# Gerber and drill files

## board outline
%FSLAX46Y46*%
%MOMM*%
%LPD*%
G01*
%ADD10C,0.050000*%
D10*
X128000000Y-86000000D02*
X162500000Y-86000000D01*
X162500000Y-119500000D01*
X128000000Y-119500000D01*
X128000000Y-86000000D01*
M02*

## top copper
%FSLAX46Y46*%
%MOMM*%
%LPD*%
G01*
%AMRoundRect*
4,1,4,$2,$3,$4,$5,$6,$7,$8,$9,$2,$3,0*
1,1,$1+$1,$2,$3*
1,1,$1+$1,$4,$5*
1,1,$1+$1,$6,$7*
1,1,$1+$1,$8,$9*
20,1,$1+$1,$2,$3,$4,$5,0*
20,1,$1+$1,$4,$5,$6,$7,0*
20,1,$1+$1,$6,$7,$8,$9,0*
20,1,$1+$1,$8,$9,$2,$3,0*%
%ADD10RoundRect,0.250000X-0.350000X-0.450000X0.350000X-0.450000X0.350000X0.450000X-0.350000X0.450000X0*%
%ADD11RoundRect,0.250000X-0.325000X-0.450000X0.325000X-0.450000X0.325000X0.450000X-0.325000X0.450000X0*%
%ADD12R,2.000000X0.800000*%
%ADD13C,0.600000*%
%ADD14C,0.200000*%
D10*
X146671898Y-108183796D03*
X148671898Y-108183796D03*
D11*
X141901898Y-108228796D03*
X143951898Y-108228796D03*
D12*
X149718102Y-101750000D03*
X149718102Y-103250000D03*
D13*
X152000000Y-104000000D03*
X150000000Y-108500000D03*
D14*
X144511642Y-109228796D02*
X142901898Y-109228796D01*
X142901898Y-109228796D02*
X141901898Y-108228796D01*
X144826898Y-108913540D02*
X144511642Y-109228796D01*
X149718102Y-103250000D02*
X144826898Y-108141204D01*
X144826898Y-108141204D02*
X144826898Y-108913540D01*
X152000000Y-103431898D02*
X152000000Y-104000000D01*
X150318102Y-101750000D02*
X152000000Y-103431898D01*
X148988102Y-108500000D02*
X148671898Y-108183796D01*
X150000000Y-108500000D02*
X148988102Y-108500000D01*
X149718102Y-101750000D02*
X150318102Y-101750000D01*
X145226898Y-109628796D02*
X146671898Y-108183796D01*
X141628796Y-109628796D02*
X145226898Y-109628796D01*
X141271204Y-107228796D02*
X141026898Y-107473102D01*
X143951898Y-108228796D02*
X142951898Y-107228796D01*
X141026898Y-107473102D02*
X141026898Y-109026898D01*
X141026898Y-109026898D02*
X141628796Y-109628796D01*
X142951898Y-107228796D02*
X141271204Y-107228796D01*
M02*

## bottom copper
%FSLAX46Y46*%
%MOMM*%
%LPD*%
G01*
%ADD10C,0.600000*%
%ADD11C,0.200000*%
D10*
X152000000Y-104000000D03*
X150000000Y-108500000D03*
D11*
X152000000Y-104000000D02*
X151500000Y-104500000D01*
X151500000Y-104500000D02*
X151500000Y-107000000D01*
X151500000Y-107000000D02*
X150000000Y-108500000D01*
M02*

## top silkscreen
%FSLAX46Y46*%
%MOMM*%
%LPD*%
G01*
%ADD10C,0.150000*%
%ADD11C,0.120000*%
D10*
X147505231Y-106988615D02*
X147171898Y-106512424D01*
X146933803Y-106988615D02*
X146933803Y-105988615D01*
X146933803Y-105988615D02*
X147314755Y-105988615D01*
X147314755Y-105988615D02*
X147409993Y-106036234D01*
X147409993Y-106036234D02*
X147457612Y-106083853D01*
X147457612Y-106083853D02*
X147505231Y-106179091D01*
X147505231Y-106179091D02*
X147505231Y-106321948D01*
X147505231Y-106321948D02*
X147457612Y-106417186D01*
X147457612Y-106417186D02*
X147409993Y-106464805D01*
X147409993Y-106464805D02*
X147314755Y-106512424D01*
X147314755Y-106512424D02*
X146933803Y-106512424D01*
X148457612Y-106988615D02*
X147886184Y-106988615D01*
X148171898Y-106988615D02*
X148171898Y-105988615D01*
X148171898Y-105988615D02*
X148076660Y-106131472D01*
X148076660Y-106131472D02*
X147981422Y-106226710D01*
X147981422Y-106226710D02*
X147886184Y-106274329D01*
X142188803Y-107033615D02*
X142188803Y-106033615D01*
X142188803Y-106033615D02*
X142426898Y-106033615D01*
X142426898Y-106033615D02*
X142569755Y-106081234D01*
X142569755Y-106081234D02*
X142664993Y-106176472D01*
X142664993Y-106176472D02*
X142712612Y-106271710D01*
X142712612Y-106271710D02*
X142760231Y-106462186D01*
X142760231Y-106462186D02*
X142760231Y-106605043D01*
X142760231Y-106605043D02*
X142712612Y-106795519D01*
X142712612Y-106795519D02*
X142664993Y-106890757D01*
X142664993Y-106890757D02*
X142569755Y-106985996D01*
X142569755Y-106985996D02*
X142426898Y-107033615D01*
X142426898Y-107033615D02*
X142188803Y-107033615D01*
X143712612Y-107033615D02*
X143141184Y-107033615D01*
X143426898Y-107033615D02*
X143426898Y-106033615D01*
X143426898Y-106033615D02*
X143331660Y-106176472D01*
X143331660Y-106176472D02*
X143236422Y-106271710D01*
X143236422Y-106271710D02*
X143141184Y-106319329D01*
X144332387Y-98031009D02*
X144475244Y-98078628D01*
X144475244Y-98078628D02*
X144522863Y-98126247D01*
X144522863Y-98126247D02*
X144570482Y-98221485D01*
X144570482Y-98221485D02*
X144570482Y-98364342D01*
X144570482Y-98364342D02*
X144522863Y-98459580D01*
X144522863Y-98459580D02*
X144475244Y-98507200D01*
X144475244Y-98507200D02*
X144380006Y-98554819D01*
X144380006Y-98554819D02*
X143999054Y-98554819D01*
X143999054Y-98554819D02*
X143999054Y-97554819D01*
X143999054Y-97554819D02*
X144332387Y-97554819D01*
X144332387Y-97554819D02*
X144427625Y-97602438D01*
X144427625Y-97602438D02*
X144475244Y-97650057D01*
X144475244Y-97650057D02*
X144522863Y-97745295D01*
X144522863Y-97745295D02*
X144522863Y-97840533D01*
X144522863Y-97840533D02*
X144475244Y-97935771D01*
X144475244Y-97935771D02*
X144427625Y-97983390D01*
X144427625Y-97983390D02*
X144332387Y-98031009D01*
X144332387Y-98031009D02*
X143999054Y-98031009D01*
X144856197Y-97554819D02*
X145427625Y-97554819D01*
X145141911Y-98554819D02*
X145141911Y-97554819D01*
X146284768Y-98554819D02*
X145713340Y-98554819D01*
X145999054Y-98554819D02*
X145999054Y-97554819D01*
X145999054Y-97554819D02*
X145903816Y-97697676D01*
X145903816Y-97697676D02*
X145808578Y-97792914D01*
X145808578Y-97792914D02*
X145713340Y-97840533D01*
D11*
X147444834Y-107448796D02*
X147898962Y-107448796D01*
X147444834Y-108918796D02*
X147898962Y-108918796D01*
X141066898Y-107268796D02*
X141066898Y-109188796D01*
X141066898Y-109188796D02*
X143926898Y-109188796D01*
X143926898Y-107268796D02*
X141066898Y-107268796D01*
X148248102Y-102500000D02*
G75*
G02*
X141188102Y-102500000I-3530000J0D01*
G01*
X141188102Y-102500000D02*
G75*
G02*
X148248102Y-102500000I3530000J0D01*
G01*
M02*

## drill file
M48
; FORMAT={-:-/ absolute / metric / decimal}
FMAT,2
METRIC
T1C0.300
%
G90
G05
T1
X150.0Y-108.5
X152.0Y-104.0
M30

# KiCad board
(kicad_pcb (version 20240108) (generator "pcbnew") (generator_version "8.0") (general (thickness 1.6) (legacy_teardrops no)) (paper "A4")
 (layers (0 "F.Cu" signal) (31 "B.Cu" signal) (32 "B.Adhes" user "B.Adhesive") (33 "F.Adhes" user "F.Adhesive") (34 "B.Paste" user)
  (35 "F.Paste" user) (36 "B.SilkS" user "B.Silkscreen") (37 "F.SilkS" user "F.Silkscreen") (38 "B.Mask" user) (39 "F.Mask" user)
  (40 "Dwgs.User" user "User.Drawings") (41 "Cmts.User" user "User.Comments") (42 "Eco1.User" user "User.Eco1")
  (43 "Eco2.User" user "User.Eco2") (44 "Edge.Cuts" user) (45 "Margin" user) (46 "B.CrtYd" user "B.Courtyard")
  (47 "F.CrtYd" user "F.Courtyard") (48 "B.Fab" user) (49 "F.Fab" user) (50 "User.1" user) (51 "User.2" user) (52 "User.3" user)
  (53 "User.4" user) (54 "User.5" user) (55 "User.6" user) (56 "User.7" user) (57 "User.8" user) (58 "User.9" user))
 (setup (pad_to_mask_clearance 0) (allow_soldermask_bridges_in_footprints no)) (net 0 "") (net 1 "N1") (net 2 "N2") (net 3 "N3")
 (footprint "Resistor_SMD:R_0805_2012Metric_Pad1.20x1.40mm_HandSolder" (layer "F.Cu") (at 147.671898 108.183796)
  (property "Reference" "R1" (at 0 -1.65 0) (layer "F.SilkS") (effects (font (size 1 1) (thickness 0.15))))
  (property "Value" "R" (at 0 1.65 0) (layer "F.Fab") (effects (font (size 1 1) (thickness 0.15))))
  (fp_line (start -0.227064 -0.735) (end 0.227064 -0.735) (stroke (width 0.12) (type solid)) (layer "F.SilkS"))
  (fp_line (start -0.227064 0.735) (end 0.227064 0.735) (stroke (width 0.12) (type solid)) (layer "F.SilkS"))
  (pad "1" smd roundrect (at -1 0) (size 1.2 1.4) (layers "F.Cu" "F.Paste" "F.Mask") (roundrect_rratio 0.208333) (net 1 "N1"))
  (pad "2" smd roundrect (at 1 0) (size 1.2 1.4) (layers "F.Cu" "F.Paste" "F.Mask") (roundrect_rratio 0.208333) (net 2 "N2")))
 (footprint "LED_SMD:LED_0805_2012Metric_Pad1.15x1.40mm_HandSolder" (layer "F.Cu") (at 142.926898 108.228796)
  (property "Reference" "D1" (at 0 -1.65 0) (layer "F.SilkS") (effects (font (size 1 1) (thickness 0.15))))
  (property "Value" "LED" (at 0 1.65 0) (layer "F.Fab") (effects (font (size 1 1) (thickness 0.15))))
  (fp_line (start -1.86 -0.96) (end -1.86 0.96) (stroke (width 0.12) (type solid)) (layer "F.SilkS"))
  (fp_line (start -1.86 0.96) (end 1 0.96) (stroke (width 0.12) (type solid)) (layer "F.SilkS"))
  (fp_line (start 1 -0.96) (end -1.86 -0.96) (stroke (width 0.12) (type solid)) (layer "F.SilkS"))
  (pad "1" smd roundrect (at -1.025 0) (size 1.15 1.4) (layers "F.Cu" "F.Paste" "F.Mask") (roundrect_rratio 0.217391) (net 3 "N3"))
  (pad "2" smd roundrect (at 1.025 0) (size 1.15 1.4) (layers "F.Cu" "F.Paste" "F.Mask") (roundrect_rratio 0.217391) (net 1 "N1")))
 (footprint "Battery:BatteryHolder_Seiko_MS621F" (layer "F.Cu") (at 149.718102 102.5)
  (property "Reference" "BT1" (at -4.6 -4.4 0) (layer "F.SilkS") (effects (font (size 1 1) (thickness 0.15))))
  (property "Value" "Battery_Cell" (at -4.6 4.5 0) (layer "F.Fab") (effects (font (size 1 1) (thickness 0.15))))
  (fp_circle (center -5 0) (end -1.47 0) (stroke (width 0.12) (type solid)) (fill none) (layer "F.SilkS"))
  (pad "1" smd rect (at 0 -0.75) (size 2 0.8) (layers "F.Cu" "F.Paste" "F.Mask") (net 2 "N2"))
  (pad "2" smd rect (at 0 0.75) (size 2 0.8) (layers "F.Cu" "F.Paste" "F.Mask") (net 3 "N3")))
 (gr_rect (start 128 86) (end 162.5 119.5) (stroke (width 0.05) (type default)) (fill none) (layer "Edge.Cuts"))
 (segment (start 144.511642 109.228796) (end 142.901898 109.228796) (width 0.2) (layer "F.Cu") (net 3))
 (segment (start 142.901898 109.228796) (end 141.901898 108.228796) (width 0.2) (layer "F.Cu") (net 3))
 (segment (start 144.826898 108.91354) (end 144.511642 109.228796) (width 0.2) (layer "F.Cu") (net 3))
 (segment (start 149.718102 103.25) (end 144.826898 108.141204) (width 0.2) (layer "F.Cu") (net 3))
 (segment (start 144.826898 108.141204) (end 144.826898 108.91354) (width 0.2) (layer "F.Cu") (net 3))
 (segment (start 152 103.431898) (end 152 104) (width 0.2) (layer "F.Cu") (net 2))
 (segment (start 150.318102 101.75) (end 152 103.431898) (width 0.2) (layer "F.Cu") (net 2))
 (segment (start 148.988102 108.5) (end 148.671898 108.183796) (width 0.2) (layer "F.Cu") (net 2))
 (segment (start 150 108.5) (end 148.988102 108.5) (width 0.2) (layer "F.Cu") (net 2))
 (segment (start 149.718102 101.75) (end 150.318102 101.75) (width 0.2) (layer "F.Cu") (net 2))
 (via (at 152 104) (size 0.6) (drill 0.3) (layers "F.Cu" "B.Cu") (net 2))
 (via (at 150 108.5) (size 0.6) (drill 0.3) (layers "F.Cu" "B.Cu") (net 2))
 (segment (start 152 104) (end 151.5 104.5) (width 0.2) (layer "B.Cu") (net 2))
 (segment (start 151.5 104.5) (end 151.5 107) (width 0.2) (layer "B.Cu") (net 2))
 (segment (start 151.5 107) (end 150 108.5) (width 0.2) (layer "B.Cu") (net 2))
 (segment (start 145.226898 109.628796) (end 146.671898 108.183796) (width 0.2) (layer "F.Cu") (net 1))
 (segment (start 141.628796 109.628796) (end 145.226898 109.628796) (width 0.2) (layer "F.Cu") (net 1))
 (segment (start 141.271204 107.228796) (end 141.026898 107.473102) (width 0.2) (layer "F.Cu") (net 1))
 (segment (start 143.951898 108.228796) (end 142.951898 107.228796) (width 0.2) (layer "F.Cu") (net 1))
 (segment (start 141.026898 107.473102) (end 141.026898 109.026898) (width 0.2) (layer "F.Cu") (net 1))
 (segment (start 141.026898 109.026898) (end 141.628796 109.628796) (width 0.2) (layer "F.Cu") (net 1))
 (segment (start 142.951898 107.228796) (end 141.271204 107.228796) (width 0.2) (layer "F.Cu") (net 1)))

